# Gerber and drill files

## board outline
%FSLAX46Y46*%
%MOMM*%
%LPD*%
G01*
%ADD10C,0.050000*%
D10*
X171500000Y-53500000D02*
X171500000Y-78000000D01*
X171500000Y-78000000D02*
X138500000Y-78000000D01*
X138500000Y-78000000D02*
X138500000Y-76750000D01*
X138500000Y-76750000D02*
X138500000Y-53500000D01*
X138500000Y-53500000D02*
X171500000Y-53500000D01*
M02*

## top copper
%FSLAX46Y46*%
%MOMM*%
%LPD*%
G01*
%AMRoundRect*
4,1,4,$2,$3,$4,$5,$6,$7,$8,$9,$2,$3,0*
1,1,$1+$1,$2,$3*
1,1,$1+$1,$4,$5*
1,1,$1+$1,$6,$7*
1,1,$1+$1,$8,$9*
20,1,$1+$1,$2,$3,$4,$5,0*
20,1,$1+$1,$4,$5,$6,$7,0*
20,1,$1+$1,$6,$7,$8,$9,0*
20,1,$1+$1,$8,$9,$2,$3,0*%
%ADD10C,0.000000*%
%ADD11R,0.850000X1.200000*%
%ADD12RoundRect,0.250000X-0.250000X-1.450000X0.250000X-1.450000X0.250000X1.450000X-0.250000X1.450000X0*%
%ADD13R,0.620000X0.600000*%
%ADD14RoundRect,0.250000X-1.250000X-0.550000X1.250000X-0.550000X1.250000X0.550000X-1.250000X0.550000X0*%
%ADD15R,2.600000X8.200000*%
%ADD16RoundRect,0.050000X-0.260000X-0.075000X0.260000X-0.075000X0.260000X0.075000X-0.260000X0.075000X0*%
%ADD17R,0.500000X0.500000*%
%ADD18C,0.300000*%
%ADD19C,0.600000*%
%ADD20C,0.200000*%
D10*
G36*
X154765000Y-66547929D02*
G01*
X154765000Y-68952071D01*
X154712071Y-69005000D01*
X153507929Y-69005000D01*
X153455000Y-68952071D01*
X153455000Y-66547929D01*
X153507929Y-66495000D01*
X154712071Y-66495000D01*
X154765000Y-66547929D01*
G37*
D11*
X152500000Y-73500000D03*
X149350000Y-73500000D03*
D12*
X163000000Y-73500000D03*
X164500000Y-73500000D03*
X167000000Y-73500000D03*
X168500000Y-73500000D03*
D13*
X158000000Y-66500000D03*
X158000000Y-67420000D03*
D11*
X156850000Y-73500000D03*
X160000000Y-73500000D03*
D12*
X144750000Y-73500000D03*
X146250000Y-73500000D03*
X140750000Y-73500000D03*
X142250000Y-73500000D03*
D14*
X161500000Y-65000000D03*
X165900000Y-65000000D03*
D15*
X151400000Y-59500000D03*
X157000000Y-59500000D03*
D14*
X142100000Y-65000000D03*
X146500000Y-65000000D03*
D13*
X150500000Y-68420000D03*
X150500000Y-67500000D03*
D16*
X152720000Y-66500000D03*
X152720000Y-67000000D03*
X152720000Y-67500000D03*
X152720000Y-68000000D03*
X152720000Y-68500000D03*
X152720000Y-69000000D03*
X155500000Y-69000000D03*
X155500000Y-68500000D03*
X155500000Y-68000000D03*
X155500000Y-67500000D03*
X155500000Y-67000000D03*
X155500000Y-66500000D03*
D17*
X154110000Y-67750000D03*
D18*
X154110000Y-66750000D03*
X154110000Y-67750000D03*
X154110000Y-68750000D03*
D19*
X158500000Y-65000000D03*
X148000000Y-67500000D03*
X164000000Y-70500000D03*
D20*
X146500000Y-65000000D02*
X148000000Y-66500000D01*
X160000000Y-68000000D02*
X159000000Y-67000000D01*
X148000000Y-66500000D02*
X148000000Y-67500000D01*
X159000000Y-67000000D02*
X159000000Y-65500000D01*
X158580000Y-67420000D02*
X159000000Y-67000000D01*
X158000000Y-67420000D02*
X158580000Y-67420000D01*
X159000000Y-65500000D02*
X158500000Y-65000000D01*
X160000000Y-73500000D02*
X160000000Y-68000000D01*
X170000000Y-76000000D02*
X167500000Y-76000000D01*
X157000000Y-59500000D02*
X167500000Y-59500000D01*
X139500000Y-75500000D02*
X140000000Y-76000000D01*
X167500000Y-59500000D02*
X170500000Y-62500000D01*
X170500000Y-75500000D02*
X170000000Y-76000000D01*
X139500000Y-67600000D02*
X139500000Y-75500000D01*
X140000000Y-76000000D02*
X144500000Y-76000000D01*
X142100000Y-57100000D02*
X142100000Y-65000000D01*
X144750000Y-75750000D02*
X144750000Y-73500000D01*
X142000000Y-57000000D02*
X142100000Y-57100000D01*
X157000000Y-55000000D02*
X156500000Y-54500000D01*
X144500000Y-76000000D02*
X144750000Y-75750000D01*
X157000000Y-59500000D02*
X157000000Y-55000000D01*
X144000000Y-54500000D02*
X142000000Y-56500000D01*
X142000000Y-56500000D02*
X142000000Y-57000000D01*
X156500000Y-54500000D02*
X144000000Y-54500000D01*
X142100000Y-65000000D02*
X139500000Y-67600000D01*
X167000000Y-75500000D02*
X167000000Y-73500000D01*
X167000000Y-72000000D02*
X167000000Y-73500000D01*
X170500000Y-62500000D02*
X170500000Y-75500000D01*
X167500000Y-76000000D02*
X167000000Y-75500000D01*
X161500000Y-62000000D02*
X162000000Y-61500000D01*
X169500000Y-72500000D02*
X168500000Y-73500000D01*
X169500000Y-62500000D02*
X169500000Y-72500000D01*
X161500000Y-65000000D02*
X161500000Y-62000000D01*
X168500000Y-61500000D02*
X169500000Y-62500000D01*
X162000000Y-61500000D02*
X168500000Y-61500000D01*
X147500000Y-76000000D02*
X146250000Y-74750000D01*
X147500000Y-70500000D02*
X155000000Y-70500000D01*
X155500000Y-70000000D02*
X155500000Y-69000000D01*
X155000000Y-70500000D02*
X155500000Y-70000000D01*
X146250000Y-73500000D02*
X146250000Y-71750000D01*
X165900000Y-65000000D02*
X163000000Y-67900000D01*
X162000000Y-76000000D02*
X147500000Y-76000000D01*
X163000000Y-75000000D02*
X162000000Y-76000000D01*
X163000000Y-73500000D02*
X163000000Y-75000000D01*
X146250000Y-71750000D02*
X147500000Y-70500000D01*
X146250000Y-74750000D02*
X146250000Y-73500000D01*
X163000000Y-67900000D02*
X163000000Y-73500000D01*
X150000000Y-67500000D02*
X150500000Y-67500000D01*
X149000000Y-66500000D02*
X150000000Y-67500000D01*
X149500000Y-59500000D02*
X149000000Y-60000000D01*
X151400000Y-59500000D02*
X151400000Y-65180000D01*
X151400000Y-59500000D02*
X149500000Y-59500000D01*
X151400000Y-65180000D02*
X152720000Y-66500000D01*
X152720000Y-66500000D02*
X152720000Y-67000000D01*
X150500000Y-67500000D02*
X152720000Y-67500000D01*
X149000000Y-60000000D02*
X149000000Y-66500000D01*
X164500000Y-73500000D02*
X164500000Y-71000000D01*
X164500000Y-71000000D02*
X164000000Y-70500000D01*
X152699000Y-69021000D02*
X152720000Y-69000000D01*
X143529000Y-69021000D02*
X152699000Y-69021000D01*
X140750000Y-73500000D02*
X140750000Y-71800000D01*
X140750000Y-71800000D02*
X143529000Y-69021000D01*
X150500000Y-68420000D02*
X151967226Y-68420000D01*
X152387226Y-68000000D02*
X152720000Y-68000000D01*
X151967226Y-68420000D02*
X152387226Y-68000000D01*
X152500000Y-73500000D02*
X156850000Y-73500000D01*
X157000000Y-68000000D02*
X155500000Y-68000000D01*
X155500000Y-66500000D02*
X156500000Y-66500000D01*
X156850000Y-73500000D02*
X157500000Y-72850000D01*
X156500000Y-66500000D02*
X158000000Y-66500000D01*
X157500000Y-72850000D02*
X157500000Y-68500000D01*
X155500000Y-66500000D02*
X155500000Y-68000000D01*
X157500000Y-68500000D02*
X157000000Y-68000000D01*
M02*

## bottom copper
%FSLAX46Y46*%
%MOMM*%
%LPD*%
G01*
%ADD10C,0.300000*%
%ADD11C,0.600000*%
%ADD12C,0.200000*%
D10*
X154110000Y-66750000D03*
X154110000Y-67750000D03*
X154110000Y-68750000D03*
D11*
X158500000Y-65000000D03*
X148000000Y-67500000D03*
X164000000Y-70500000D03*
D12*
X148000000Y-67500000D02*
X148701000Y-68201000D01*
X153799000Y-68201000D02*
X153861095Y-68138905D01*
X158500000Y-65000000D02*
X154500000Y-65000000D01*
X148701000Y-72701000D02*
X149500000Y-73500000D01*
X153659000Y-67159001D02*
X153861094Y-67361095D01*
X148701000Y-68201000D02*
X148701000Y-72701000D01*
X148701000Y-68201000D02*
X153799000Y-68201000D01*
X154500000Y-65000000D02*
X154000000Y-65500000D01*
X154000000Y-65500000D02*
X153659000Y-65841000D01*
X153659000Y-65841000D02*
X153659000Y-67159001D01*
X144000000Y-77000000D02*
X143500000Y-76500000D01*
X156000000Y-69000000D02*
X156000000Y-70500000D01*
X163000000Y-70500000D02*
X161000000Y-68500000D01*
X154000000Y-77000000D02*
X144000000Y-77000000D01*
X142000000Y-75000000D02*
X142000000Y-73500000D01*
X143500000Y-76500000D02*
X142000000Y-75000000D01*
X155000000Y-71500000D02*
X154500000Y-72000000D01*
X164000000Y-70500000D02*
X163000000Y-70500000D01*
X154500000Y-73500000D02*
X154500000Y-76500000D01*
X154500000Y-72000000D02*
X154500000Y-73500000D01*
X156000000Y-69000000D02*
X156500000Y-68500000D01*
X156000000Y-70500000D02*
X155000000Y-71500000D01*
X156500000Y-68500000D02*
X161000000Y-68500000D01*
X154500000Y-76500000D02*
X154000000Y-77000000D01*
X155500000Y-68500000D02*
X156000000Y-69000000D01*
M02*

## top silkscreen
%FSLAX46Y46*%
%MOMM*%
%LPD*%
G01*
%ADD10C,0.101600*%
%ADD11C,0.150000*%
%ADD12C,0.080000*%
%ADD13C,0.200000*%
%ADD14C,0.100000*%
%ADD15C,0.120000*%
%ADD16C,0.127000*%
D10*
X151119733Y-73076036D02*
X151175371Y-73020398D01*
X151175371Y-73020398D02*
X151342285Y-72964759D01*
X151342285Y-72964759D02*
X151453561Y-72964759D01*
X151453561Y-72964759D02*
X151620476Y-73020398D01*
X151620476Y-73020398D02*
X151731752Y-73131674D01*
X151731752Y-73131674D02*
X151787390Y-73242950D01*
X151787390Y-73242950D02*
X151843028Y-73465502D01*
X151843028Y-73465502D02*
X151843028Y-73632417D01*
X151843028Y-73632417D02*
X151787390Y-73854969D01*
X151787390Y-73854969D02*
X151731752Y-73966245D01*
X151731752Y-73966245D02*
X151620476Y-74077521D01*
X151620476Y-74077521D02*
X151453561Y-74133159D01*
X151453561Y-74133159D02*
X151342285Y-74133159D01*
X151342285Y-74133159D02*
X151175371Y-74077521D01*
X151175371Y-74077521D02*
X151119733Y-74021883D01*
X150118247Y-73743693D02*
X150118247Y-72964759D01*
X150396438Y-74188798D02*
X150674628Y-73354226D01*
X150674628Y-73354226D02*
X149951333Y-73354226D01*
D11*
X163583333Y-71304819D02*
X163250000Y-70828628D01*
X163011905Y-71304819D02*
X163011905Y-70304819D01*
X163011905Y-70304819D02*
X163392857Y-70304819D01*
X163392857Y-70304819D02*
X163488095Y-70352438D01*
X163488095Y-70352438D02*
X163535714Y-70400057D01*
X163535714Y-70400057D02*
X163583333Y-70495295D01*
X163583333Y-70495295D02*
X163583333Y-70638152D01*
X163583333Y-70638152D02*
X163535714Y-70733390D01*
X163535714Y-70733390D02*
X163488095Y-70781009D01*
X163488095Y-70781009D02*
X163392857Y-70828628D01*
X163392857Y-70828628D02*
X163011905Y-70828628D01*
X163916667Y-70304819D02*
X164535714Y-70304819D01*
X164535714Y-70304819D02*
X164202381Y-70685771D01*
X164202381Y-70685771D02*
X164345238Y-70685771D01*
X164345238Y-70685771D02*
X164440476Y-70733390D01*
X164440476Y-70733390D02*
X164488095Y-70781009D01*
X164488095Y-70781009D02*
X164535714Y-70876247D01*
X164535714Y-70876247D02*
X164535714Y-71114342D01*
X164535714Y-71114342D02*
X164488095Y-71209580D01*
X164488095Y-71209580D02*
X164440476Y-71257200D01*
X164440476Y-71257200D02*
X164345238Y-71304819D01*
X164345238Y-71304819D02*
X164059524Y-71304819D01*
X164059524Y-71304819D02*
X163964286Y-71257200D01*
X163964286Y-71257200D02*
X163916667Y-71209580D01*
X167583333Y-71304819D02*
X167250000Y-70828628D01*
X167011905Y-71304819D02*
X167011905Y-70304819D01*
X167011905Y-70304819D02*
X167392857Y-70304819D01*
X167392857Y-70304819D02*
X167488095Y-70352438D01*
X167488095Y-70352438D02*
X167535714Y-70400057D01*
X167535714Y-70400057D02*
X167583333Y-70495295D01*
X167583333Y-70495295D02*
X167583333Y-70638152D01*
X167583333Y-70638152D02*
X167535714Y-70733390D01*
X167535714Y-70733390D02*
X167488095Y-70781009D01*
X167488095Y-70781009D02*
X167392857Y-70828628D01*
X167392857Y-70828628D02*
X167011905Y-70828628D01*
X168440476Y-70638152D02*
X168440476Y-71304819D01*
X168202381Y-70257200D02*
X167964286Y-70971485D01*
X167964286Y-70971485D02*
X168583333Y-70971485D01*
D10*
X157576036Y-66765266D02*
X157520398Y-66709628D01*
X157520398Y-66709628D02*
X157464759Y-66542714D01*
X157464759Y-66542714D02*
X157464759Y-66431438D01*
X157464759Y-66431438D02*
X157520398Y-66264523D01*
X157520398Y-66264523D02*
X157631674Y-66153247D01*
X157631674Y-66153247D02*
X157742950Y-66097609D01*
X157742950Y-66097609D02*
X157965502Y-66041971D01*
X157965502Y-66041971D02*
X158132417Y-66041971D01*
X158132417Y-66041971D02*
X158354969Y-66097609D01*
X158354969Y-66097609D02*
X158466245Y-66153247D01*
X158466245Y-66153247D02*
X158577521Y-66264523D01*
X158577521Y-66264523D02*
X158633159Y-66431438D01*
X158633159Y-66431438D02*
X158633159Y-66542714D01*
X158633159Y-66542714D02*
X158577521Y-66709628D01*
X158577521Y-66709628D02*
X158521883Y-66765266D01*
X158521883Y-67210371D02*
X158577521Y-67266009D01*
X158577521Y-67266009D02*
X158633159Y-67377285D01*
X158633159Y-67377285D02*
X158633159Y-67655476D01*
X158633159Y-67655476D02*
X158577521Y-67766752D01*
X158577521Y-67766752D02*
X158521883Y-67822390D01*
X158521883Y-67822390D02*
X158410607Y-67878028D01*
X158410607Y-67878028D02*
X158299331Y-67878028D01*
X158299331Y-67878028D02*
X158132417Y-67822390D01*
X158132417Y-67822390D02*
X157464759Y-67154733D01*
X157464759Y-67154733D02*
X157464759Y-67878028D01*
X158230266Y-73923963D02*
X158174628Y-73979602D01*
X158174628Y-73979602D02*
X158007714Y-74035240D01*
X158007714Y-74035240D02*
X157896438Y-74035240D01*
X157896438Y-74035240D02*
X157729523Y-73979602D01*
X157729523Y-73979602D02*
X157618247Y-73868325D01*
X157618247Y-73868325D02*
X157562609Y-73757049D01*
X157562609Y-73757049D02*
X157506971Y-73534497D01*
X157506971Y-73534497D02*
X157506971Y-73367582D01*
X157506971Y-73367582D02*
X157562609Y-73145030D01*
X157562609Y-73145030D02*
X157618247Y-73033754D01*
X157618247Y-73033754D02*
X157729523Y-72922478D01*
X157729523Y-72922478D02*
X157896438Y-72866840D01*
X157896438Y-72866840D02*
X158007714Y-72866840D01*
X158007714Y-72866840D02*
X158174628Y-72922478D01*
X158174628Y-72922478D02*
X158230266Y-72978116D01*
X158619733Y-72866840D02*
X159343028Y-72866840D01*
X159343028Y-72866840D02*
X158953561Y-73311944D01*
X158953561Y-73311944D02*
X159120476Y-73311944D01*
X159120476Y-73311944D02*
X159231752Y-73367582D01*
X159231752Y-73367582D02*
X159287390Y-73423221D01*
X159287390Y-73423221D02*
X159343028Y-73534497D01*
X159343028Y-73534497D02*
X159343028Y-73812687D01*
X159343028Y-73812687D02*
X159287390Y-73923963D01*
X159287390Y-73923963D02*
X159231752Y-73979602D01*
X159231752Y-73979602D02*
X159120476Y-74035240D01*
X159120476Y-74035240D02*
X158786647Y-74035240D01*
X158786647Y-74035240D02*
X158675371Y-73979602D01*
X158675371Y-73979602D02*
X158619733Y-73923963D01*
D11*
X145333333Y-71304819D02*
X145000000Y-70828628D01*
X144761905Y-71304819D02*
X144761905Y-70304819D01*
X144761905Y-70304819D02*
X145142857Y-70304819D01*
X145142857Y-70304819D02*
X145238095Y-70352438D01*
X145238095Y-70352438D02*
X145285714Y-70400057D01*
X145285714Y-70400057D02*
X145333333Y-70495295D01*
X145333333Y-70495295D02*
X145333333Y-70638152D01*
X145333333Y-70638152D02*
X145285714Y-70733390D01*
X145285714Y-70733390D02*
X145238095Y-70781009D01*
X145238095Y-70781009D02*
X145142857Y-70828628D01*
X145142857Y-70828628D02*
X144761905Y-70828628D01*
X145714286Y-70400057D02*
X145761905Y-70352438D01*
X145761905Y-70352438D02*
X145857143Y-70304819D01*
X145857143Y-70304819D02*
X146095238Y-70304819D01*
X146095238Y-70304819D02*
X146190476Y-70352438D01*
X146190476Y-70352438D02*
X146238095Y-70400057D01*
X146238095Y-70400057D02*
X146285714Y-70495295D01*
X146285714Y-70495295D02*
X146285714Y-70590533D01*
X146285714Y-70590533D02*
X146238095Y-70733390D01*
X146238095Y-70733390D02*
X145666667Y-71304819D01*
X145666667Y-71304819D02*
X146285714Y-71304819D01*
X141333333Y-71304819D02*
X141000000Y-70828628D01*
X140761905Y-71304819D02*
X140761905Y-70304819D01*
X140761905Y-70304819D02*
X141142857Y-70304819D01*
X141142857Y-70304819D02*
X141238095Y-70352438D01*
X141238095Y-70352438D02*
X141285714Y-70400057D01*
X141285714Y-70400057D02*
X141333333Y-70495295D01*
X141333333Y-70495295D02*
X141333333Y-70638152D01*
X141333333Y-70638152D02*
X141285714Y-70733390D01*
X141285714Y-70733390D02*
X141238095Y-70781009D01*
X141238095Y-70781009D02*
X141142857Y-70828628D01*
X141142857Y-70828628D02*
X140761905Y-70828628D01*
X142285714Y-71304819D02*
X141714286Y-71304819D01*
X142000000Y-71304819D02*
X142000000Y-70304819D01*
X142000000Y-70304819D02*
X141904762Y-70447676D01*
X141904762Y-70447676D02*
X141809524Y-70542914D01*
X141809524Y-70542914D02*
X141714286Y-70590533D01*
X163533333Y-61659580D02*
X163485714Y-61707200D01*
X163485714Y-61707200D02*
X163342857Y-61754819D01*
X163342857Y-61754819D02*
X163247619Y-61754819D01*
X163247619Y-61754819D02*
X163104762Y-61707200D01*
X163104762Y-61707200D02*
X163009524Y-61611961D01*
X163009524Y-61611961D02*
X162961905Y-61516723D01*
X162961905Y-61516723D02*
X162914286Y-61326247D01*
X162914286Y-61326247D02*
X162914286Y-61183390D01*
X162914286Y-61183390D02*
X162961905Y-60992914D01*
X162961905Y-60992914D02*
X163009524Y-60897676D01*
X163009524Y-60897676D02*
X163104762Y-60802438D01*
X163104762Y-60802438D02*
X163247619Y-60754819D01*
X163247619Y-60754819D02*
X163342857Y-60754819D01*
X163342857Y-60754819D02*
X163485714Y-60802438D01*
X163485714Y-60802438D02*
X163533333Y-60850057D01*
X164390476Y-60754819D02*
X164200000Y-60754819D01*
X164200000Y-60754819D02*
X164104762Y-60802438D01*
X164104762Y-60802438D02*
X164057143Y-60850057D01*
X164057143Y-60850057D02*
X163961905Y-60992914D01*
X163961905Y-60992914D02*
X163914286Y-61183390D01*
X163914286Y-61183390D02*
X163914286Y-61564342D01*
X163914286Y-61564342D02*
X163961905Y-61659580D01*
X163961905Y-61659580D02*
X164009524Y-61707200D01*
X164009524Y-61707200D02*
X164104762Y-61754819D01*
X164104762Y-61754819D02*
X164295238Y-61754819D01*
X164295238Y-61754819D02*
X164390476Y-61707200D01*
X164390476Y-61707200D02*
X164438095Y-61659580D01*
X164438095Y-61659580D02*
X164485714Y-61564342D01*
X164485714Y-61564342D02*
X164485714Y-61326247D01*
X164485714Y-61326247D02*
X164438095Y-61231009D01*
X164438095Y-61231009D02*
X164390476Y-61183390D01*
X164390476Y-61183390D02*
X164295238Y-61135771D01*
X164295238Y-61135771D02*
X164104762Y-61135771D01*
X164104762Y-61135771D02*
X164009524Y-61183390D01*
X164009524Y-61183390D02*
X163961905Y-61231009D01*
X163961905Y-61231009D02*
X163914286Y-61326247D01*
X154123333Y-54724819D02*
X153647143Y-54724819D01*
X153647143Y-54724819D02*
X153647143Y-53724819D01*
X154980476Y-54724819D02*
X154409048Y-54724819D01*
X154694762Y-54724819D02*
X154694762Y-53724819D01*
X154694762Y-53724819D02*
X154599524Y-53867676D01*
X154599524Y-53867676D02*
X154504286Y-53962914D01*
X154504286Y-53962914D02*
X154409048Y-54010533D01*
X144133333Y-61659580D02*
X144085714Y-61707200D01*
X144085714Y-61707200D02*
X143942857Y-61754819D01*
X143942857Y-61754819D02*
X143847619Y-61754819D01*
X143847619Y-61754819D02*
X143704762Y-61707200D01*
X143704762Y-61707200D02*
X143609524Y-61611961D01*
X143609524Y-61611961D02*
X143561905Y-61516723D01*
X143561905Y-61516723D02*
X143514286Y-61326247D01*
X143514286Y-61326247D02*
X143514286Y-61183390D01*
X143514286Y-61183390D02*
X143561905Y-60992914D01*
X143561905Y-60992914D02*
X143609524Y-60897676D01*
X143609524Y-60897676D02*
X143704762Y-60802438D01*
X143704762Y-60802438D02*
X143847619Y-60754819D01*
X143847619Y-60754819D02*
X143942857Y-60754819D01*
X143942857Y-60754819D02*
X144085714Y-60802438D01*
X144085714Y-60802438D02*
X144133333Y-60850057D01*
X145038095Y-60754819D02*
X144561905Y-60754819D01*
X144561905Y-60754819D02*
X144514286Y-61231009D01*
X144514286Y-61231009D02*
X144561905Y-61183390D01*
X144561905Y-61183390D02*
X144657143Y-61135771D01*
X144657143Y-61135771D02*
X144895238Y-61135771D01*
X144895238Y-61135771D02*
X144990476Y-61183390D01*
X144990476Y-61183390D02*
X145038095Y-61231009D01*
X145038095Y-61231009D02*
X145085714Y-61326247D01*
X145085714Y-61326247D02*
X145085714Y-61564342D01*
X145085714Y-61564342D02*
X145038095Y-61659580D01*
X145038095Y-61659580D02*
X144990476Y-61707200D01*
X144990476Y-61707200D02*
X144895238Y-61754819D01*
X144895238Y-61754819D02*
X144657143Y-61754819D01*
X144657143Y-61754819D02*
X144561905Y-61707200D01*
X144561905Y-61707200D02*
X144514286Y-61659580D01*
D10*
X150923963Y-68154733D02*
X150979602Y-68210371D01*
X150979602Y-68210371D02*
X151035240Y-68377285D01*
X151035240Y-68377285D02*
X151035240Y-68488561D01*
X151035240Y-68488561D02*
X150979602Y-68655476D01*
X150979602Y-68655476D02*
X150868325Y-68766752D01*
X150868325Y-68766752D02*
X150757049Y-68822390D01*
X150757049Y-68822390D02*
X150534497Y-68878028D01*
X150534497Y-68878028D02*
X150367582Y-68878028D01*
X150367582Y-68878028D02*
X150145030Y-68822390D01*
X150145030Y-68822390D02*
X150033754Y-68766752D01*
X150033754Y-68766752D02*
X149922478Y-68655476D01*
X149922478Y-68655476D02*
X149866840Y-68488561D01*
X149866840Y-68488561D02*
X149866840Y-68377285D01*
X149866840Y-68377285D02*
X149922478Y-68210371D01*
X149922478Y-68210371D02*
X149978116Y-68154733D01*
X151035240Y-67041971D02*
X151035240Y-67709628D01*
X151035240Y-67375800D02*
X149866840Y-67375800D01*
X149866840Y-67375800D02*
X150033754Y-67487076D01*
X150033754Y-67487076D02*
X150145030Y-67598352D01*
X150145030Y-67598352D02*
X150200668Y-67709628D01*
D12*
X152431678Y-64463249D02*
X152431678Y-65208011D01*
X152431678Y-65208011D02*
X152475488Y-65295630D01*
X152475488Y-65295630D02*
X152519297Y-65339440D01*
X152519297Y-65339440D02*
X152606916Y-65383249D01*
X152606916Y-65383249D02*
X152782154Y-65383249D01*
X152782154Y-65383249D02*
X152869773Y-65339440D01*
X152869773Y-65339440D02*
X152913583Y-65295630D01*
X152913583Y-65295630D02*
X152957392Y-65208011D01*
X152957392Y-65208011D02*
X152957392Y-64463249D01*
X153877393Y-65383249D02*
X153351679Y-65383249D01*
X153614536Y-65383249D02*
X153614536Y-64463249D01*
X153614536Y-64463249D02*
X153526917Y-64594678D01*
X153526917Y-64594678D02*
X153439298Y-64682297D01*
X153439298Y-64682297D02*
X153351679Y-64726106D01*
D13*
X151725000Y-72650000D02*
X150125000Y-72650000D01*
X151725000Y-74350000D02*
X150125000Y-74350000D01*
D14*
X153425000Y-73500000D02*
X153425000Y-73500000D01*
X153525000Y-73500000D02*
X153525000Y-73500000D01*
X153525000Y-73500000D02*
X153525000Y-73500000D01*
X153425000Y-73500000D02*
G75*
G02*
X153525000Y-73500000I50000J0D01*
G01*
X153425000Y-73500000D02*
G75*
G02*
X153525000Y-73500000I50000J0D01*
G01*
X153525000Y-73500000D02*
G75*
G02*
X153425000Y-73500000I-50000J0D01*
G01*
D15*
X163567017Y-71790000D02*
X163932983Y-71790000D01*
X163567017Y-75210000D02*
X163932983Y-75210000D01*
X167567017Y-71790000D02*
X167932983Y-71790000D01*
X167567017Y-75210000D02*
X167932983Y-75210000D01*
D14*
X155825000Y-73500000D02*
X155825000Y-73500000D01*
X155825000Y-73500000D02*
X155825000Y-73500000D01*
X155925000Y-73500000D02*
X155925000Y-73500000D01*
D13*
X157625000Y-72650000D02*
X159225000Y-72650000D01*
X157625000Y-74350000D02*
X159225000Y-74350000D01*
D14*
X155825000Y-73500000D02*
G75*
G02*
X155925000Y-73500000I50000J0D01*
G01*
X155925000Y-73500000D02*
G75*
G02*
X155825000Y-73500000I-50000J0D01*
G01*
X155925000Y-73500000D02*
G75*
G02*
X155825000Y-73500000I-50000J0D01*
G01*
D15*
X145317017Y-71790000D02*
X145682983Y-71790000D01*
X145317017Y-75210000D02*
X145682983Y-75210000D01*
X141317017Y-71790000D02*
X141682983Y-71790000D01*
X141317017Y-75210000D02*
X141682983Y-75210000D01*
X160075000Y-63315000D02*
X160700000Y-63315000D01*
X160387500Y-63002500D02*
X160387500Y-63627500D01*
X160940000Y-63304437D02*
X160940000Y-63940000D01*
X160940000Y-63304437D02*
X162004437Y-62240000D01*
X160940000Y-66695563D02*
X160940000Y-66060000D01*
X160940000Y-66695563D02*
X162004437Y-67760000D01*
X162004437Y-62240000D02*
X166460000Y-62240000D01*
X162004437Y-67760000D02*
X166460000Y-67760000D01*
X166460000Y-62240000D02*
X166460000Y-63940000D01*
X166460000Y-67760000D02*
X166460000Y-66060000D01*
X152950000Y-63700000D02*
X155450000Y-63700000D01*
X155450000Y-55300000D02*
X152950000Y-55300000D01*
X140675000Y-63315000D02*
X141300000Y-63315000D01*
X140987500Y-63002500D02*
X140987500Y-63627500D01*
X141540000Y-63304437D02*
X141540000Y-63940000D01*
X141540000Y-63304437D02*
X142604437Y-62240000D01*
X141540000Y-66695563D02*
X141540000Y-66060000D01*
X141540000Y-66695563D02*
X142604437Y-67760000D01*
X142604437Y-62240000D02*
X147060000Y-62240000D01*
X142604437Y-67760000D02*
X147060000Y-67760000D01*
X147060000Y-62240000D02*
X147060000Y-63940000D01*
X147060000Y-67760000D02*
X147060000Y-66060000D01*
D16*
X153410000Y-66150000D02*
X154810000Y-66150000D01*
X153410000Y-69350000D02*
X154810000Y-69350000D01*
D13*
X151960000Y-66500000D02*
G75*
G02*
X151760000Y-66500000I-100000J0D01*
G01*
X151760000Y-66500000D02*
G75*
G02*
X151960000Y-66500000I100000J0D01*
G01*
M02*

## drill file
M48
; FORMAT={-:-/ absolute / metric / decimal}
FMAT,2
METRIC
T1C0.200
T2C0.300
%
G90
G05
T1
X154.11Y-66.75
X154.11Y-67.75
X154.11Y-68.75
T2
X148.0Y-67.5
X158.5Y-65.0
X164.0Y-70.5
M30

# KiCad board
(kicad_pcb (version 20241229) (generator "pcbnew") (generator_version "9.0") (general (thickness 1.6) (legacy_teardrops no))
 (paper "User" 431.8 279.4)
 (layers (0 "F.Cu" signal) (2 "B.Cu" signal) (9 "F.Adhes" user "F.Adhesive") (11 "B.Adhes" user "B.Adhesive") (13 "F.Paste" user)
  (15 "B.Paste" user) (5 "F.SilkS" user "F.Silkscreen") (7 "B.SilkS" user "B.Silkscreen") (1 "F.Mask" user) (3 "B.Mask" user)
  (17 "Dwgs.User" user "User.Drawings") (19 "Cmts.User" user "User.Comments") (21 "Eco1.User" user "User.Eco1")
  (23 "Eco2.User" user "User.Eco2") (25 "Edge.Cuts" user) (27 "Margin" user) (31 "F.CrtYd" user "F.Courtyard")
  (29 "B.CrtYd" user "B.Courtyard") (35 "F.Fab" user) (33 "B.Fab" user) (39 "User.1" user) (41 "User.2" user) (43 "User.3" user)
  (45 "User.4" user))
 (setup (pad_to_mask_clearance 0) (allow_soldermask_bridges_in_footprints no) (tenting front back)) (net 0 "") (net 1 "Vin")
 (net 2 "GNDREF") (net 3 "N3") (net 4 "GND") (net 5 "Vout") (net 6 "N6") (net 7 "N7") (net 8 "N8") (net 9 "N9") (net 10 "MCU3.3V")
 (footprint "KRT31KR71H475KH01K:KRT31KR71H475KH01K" (layer "F.Cu") (at 150.925 73.5 180)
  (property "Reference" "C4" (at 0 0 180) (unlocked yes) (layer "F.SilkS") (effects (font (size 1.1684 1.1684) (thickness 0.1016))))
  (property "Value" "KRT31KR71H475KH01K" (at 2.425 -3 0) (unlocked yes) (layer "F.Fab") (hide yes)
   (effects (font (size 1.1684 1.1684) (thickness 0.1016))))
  (fp_line (start -0.8 0.85) (end 0.8 0.85) (stroke (width 0.2) (type solid)) (layer "F.SilkS"))
  (fp_line (start -0.8 -0.85) (end 0.8 -0.85) (stroke (width 0.2) (type solid)) (layer "F.SilkS"))
  (fp_line (start -2.5 0) (end -2.5 0) (stroke (width 0.1) (type solid)) (layer "F.SilkS"))
  (fp_line (start -2.6 0) (end -2.6 0) (stroke (width 0.1) (type solid)) (layer "F.SilkS"))
  (fp_line (start -2.6 0) (end -2.6 0) (stroke (width 0.1) (type solid)) (layer "F.SilkS"))
  (fp_arc (start -2.5 0) (mid -2.55 0.05) (end -2.6 0) (stroke (width 0.1) (type solid)) (layer "F.SilkS"))
  (fp_arc (start -2.5 0) (mid -2.55 0.05) (end -2.6 0) (stroke (width 0.1) (type solid)) (layer "F.SilkS"))
  (fp_arc (start -2.6 0) (mid -2.55 -0.05) (end -2.5 0) (stroke (width 0.1) (type solid)) (layer "F.SilkS"))
  (pad "1" smd rect (at -1.575 0 270) (size 1.2 0.85) (layers "F.Cu" "F.Mask" "F.Paste") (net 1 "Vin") (solder_mask_margin 0.1016)
   (solder_paste_margin 0) (thermal_bridge_angle 0))
  (pad "2" smd rect (at 1.575 0 270) (size 1.2 0.85) (layers "F.Cu" "F.Mask" "F.Paste") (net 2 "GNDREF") (solder_mask_margin 0.1016)
   (solder_paste_margin 0) (thermal_bridge_angle 0)))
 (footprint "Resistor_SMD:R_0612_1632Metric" (layer "F.Cu") (at 163.75 73.5)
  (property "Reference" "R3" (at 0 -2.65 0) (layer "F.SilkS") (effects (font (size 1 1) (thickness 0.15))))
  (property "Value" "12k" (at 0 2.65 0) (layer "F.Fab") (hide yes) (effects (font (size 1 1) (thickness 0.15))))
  (fp_line (start -0.182983 -1.71) (end 0.182983 -1.71) (stroke (width 0.12) (type solid)) (layer "F.SilkS"))
  (fp_line (start -0.182983 1.71) (end 0.182983 1.71) (stroke (width 0.12) (type solid)) (layer "F.SilkS"))
  (pad "1" smd roundrect (at -0.75 0) (size 1 3.4) (layers "F.Cu" "F.Mask" "F.Paste") (roundrect_rratio 0.25) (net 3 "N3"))
  (pad "2" smd roundrect (at 0.75 0) (size 1 3.4) (layers "F.Cu" "F.Mask" "F.Paste") (roundrect_rratio 0.25) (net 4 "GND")))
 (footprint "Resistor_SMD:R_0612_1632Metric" (layer "F.Cu") (at 167.75 73.5)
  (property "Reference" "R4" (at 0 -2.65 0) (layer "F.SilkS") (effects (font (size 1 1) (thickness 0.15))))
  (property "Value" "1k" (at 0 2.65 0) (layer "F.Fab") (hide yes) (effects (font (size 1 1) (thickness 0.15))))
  (fp_line (start -0.182983 -1.71) (end 0.182983 -1.71) (stroke (width 0.12) (type solid)) (layer "F.SilkS"))
  (fp_line (start -0.182983 1.71) (end 0.182983 1.71) (stroke (width 0.12) (type solid)) (layer "F.SilkS"))
  (pad "1" smd roundrect (at -0.75 0) (size 1 3.4) (layers "F.Cu" "F.Mask" "F.Paste") (roundrect_rratio 0.25) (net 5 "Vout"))
  (pad "2" smd roundrect (at 0.75 0) (size 1 3.4) (layers "F.Cu" "F.Mask" "F.Paste") (roundrect_rratio 0.25) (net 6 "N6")))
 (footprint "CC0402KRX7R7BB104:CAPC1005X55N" (layer "F.Cu") (at 158 66.96 -90)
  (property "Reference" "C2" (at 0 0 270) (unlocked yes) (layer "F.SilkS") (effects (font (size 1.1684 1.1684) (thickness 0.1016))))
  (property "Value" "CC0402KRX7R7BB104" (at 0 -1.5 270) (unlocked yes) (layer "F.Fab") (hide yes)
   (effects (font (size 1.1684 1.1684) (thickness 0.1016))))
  (pad "1" smd rect (at -0.46 0) (size 0.62 0.6) (layers "F.Cu" "F.Mask" "F.Paste") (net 1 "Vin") (solder_mask_margin 0.1016)
   (solder_paste_margin 0) (thermal_bridge_angle 0))
  (pad "2" smd rect (at 0.46 0) (size 0.62 0.6) (layers "F.Cu" "F.Mask" "F.Paste") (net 2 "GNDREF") (solder_mask_margin 0.1016)
   (solder_paste_margin 0) (thermal_bridge_angle 0)))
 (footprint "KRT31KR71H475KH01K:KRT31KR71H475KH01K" (layer "F.Cu") (at 158.425 73.5)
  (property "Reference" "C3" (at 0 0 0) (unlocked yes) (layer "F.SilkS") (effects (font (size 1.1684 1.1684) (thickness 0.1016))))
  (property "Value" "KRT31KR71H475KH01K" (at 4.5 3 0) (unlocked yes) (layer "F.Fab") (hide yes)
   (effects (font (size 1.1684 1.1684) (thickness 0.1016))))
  (fp_line (start -2.6 0) (end -2.6 0) (stroke (width 0.1) (type solid)) (layer "F.SilkS"))
  (fp_line (start -2.6 0) (end -2.6 0) (stroke (width 0.1) (type solid)) (layer "F.SilkS"))
  (fp_line (start -2.5 0) (end -2.5 0) (stroke (width 0.1) (type solid)) (layer "F.SilkS"))
  (fp_line (start -0.8 -0.85) (end 0.8 -0.85) (stroke (width 0.2) (type solid)) (layer "F.SilkS"))
  (fp_line (start -0.8 0.85) (end 0.8 0.85) (stroke (width 0.2) (type solid)) (layer "F.SilkS"))
  (fp_arc (start -2.6 0) (mid -2.55 -0.05) (end -2.5 0) (stroke (width 0.1) (type solid)) (layer "F.SilkS"))
  (fp_arc (start -2.5 0) (mid -2.55 0.05) (end -2.6 0) (stroke (width 0.1) (type solid)) (layer "F.SilkS"))
  (fp_arc (start -2.5 0) (mid -2.55 0.05) (end -2.6 0) (stroke (width 0.1) (type solid)) (layer "F.SilkS"))
  (pad "1" smd rect (at -1.575 0 90) (size 1.2 0.85) (layers "F.Cu" "F.Mask" "F.Paste") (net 1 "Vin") (solder_mask_margin 0.1016)
   (solder_paste_margin 0) (thermal_bridge_angle 0))
  (pad "2" smd rect (at 1.575 0 90) (size 1.2 0.85) (layers "F.Cu" "F.Mask" "F.Paste") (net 2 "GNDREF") (solder_mask_margin 0.1016)
   (solder_paste_margin 0) (thermal_bridge_angle 0)))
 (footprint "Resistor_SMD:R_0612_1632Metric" (layer "F.Cu") (at 145.5 73.5)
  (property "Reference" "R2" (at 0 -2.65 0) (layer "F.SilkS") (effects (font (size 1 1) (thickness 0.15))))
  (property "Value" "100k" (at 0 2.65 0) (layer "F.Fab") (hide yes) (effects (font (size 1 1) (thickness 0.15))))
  (fp_line (start -0.182983 -1.71) (end 0.182983 -1.71) (stroke (width 0.12) (type solid)) (layer "F.SilkS"))
  (fp_line (start -0.182983 1.71) (end 0.182983 1.71) (stroke (width 0.12) (type solid)) (layer "F.SilkS"))
  (pad "1" smd roundrect (at -0.75 0) (size 1 3.4) (layers "F.Cu" "F.Mask" "F.Paste") (roundrect_rratio 0.25) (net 5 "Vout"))
  (pad "2" smd roundrect (at 0.75 0) (size 1 3.4) (layers "F.Cu" "F.Mask" "F.Paste") (roundrect_rratio 0.25) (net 3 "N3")))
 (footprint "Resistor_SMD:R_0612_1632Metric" (layer "F.Cu") (at 141.5 73.5)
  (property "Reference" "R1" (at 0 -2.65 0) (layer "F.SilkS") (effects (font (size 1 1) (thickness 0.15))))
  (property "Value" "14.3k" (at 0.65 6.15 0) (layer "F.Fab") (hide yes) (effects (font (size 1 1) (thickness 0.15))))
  (fp_line (start -0.182983 -1.71) (end 0.182983 -1.71) (stroke (width 0.12) (type solid)) (layer "F.SilkS"))
  (fp_line (start -0.182983 1.71) (end 0.182983 1.71) (stroke (width 0.12) (type solid)) (layer "F.SilkS"))
  (pad "1" smd roundrect (at -0.75 0) (size 1 3.4) (layers "F.Cu" "F.Mask" "F.Paste") (roundrect_rratio 0.25) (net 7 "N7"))
  (pad "2" smd roundrect (at 0.75 0) (size 1 3.4) (layers "F.Cu" "F.Mask" "F.Paste") (roundrect_rratio 0.25) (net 4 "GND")))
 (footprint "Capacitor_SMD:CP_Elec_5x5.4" (layer "F.Cu") (at 163.7 65)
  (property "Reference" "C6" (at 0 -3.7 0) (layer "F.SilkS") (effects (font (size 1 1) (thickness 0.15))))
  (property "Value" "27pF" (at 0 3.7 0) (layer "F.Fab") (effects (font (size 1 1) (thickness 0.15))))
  (fp_line (start -3.625 -1.685) (end -3 -1.685) (stroke (width 0.12) (type solid)) (layer "F.SilkS"))
  (fp_line (start -3.3125 -1.9975) (end -3.3125 -1.3725) (stroke (width 0.12) (type solid)) (layer "F.SilkS"))
  (fp_line (start -2.76 -1.695563) (end -2.76 -1.06) (stroke (width 0.12) (type solid)) (layer "F.SilkS"))
  (fp_line (start -2.76 -1.695563) (end -1.695563 -2.76) (stroke (width 0.12) (type solid)) (layer "F.SilkS"))
  (fp_line (start -2.76 1.695563) (end -2.76 1.06) (stroke (width 0.12) (type solid)) (layer "F.SilkS"))
  (fp_line (start -2.76 1.695563) (end -1.695563 2.76) (stroke (width 0.12) (type solid)) (layer "F.SilkS"))
  (fp_line (start -1.695563 -2.76) (end 2.76 -2.76) (stroke (width 0.12) (type solid)) (layer "F.SilkS"))
  (fp_line (start -1.695563 2.76) (end 2.76 2.76) (stroke (width 0.12) (type solid)) (layer "F.SilkS"))
  (fp_line (start 2.76 -2.76) (end 2.76 -1.06) (stroke (width 0.12) (type solid)) (layer "F.SilkS"))
  (fp_line (start 2.76 2.76) (end 2.76 1.06) (stroke (width 0.12) (type solid)) (layer "F.SilkS"))
  (pad "1" smd roundrect (at -2.2 0) (size 3 1.6) (layers "F.Cu" "F.Mask" "F.Paste") (roundrect_rratio 0.15625) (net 6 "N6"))
  (pad "2" smd roundrect (at 2.2 0) (size 3 1.6) (layers "F.Cu" "F.Mask" "F.Paste") (roundrect_rratio 0.15625) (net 3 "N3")))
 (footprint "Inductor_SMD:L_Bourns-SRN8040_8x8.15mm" (layer "F.Cu") (at 154.2 59.5)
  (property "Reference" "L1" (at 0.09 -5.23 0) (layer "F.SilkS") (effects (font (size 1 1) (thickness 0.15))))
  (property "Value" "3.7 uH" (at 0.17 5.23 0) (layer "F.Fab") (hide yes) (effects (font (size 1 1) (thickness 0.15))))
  (fp_line (start -1.25 4.2) (end 1.25 4.2) (stroke (width 0.12) (type solid)) (layer "F.SilkS"))
  (fp_line (start 1.25 -4.2) (end -1.25 -4.2) (stroke (width 0.12) (type solid)) (layer "F.SilkS"))
  (pad "1" smd rect (at -2.8 0) (size 2.6 8.2) (layers "F.Cu" "F.Mask" "F.Paste") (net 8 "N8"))
  (pad "2" smd rect (at 2.8 0) (size 2.6 8.2) (layers "F.Cu" "F.Mask" "F.Paste") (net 5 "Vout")))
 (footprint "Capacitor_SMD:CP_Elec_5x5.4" (layer "F.Cu") (at 144.3 65)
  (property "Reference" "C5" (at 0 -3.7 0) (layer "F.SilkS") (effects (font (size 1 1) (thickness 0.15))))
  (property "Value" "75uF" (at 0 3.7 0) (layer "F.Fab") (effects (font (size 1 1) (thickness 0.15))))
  (fp_line (start -3.625 -1.685) (end -3 -1.685) (stroke (width 0.12) (type solid)) (layer "F.SilkS"))
  (fp_line (start -3.3125 -1.9975) (end -3.3125 -1.3725) (stroke (width 0.12) (type solid)) (layer "F.SilkS"))
  (fp_line (start -2.76 -1.695563) (end -2.76 -1.06) (stroke (width 0.12) (type solid)) (layer "F.SilkS"))
  (fp_line (start -2.76 -1.695563) (end -1.695563 -2.76) (stroke (width 0.12) (type solid)) (layer "F.SilkS"))
  (fp_line (start -2.76 1.695563) (end -2.76 1.06) (stroke (width 0.12) (type solid)) (layer "F.SilkS"))
  (fp_line (start -2.76 1.695563) (end -1.695563 2.76) (stroke (width 0.12) (type solid)) (layer "F.SilkS"))
  (fp_line (start -1.695563 -2.76) (end 2.76 -2.76) (stroke (width 0.12) (type solid)) (layer "F.SilkS"))
  (fp_line (start -1.695563 2.76) (end 2.76 2.76) (stroke (width 0.12) (type solid)) (layer "F.SilkS"))
  (fp_line (start 2.76 -2.76) (end 2.76 -1.06) (stroke (width 0.12) (type solid)) (layer "F.SilkS"))
  (fp_line (start 2.76 2.76) (end 2.76 1.06) (stroke (width 0.12) (type solid)) (layer "F.SilkS"))
  (pad "1" smd roundrect (at -2.2 0) (size 3 1.6) (layers "F.Cu" "F.Mask" "F.Paste") (roundrect_rratio 0.15625) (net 5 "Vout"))
  (pad "2" smd roundrect (at 2.2 0) (size 3 1.6) (layers "F.Cu" "F.Mask" "F.Paste") (roundrect_rratio 0.15625) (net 2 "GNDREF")))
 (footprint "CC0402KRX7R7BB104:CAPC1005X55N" (layer "F.Cu") (at 150.5 67.96 90)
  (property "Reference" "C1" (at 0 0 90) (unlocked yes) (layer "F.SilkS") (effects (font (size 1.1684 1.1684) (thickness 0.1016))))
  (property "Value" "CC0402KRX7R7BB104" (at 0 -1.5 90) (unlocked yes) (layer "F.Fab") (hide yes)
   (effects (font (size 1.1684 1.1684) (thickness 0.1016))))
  (pad "1" smd rect (at -0.46 0 180) (size 0.62 0.6) (layers "F.Cu" "F.Mask" "F.Paste") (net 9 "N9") (solder_mask_margin 0.1016)
   (solder_paste_margin 0) (thermal_bridge_angle 0))
  (pad "2" smd rect (at 0.46 0 180) (size 0.62 0.6) (layers "F.Cu" "F.Mask" "F.Paste") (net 8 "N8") (solder_mask_margin 0.1016)
   (solder_paste_margin 0) (thermal_bridge_angle 0)))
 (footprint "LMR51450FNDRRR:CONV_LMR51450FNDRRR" (layer "F.Cu") (at 154.11 67.75)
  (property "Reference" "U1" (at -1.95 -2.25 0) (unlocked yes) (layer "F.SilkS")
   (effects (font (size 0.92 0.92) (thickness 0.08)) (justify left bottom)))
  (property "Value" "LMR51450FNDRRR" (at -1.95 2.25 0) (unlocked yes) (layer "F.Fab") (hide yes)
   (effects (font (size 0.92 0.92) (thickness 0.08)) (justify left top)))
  (fp_poly
   (pts (xy 0.655 -1.202071) (xy 0.655 1.202071) (xy 0.602071 1.255) (xy -0.602071 1.255) (xy -0.655 1.202071) (xy -0.655 -1.202071)
    (xy -0.602071 -1.255) (xy 0.602071 -1.255))
   (stroke (width 0) (type default)) (fill yes) (layer "F.Cu"))
  (fp_line (start -0.7 -1.6) (end 0.7 -1.6) (stroke (width 0.127) (type solid)) (layer "F.SilkS"))
  (fp_line (start -0.7 1.6) (end 0.7 1.6) (stroke (width 0.127) (type solid)) (layer "F.SilkS"))
  (fp_circle (center -2.25 -1.25) (end -2.15 -1.25) (stroke (width 0.2) (type solid)) (fill no) (layer "F.SilkS"))
  (pad "1" smd roundrect (at -1.39 -1.25) (size 0.62 0.25) (layers "F.Cu" "F.Paste") (roundrect_rratio 0.2) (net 8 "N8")
   (solder_mask_margin 0.1016) (solder_paste_margin 0) (thermal_bridge_angle 0))
  (pad "2" smd roundrect (at -1.39 -0.75) (size 0.62 0.25) (layers "F.Cu" "F.Paste") (roundrect_rratio 0.2) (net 8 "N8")
   (solder_mask_margin 0.1016) (solder_paste_margin 0) (thermal_bridge_angle 0))
  (pad "3" smd roundrect (at -1.39 -0.25) (size 0.62 0.25) (layers "F.Cu" "F.Paste") (roundrect_rratio 0.2) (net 8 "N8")
   (solder_mask_margin 0.1016) (solder_paste_margin 0) (thermal_bridge_angle 0))
  (pad "4" smd roundrect (at -1.39 0.25) (size 0.62 0.25) (layers "F.Cu" "F.Paste") (roundrect_rratio 0.2) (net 9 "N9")
   (solder_mask_margin 0.1016) (solder_paste_margin 0) (thermal_bridge_angle 0))
  (pad "5" smd roundrect (at -1.39 0.75) (size 0.62 0.25) (layers "F.Cu" "F.Paste") (roundrect_rratio 0.2) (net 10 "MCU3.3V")
   (solder_mask_margin 0.1016) (solder_paste_margin 0) (thermal_bridge_angle 0))
  (pad "6" smd roundrect (at -1.39 1.25) (size 0.62 0.25) (layers "F.Cu" "F.Paste") (roundrect_rratio 0.2) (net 7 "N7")
   (solder_mask_margin 0.1016) (solder_paste_margin 0) (thermal_bridge_angle 0))
  (pad "7" smd roundrect (at 1.39 1.25) (size 0.62 0.25) (layers "F.Cu" "F.Paste") (roundrect_rratio 0.2) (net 3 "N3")
   (solder_mask_margin 0.1016) (solder_paste_margin 0) (thermal_bridge_angle 0))
  (pad "8" smd roundrect (at 1.39 0.75) (size 0.62 0.25) (layers "F.Cu" "F.Paste") (roundrect_rratio 0.2) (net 4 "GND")
   (solder_mask_margin 0.1016) (solder_paste_margin 0) (thermal_bridge_angle 0))
  (pad "9" smd roundrect (at 1.39 0.25) (size 0.62 0.25) (layers "F.Cu" "F.Paste") (roundrect_rratio 0.2) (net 1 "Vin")
   (solder_mask_margin 0.1016) (solder_paste_margin 0) (thermal_bridge_angle 0))
  (pad "10" smd roundrect (at 1.39 -0.25) (size 0.62 0.25) (layers "F.Cu" "F.Paste") (roundrect_rratio 0.2) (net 1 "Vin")
   (solder_mask_margin 0.1016) (solder_paste_margin 0) (thermal_bridge_angle 0))
  (pad "11" smd roundrect (at 1.39 -0.75) (size 0.62 0.25) (layers "F.Cu" "F.Paste") (roundrect_rratio 0.2) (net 1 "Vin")
   (solder_mask_margin 0.1016) (solder_paste_margin 0) (thermal_bridge_angle 0))
  (pad "12" smd roundrect (at 1.39 -1.25) (size 0.62 0.25) (layers "F.Cu" "F.Paste") (roundrect_rratio 0.2) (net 1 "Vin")
   (solder_mask_margin 0.1016) (solder_paste_margin 0) (thermal_bridge_angle 0))
  (pad "13" smd rect (at 0 0) (size 0.5 0.5) (layers "F.Cu") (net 2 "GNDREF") (solder_mask_margin 0.1016) (solder_paste_margin 0)
   (thermal_bridge_angle 0))
  (pad "14" thru_hole circle (at 0 -1) (size 0.3 0.3) (drill 0.2) (layers "*.Cu") (remove_unused_layers no) (solder_mask_margin 0.1016)
   (thermal_bridge_angle 0))
  (pad "15" thru_hole circle (at 0 0) (size 0.3 0.3) (drill 0.2) (layers "*.Cu") (remove_unused_layers no) (solder_mask_margin 0.1016)
   (thermal_bridge_angle 0))
  (pad "16" thru_hole circle (at 0 1) (size 0.3 0.3) (drill 0.2) (layers "*.Cu") (remove_unused_layers no) (solder_mask_margin 0.1016)
   (thermal_bridge_angle 0)))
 (gr_line (start 171.5 53.5) (end 171.5 78) (stroke (width 0.05) (type default)) (layer "Edge.Cuts"))
 (gr_line (start 171.5 78) (end 138.5 78) (stroke (width 0.05) (type default)) (layer "Edge.Cuts"))
 (gr_line (start 138.5 78) (end 138.5 76.75) (stroke (width 0.05) (type default)) (layer "Edge.Cuts"))
 (gr_line (start 138.5 76.75) (end 138.5 53.5) (stroke (width 0.05) (type default)) (layer "Edge.Cuts"))
 (gr_line (start 138.5 53.5) (end 171.5 53.5) (stroke (width 0.05) (type default)) (layer "Edge.Cuts"))
 (segment (start 146.5 65) (end 148 66.5) (width 0.2) (layer "F.Cu") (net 2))
 (segment (start 160 68) (end 159 67) (width 0.2) (layer "F.Cu") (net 2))
 (segment (start 148 66.5) (end 148 67.5) (width 0.2) (layer "F.Cu") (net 2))
 (segment (start 159 67) (end 159 65.5) (width 0.2) (layer "F.Cu") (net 2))
 (segment (start 158.58 67.42) (end 159 67) (width 0.2) (layer "F.Cu") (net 2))
 (segment (start 158 67.42) (end 158.58 67.42) (width 0.2) (layer "F.Cu") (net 2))
 (segment (start 159 65.5) (end 158.5 65) (width 0.2) (layer "F.Cu") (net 2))
 (segment (start 160 73.5) (end 160 68) (width 0.2) (layer "F.Cu") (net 2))
 (via (at 158.5 65) (size 0.6) (drill 0.3) (layers "F.Cu" "B.Cu") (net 2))
 (via (at 148 67.5) (size 0.6) (drill 0.3) (layers "F.Cu" "B.Cu") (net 2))
 (segment (start 148 67.5) (end 148.701 68.201) (width 0.2) (layer "B.Cu") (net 2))
 (segment (start 153.799 68.201) (end 153.861095 68.138905) (width 0.2) (layer "B.Cu") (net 2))
 (segment (start 158.5 65) (end 154.5 65) (width 0.2) (layer "B.Cu") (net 2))
 (segment (start 148.701 72.701) (end 149.5 73.5) (width 0.2) (layer "B.Cu") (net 2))
 (segment (start 153.659 67.159001) (end 153.861094 67.361095) (width 0.2) (layer "B.Cu") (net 2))
 (segment (start 148.701 68.201) (end 148.701 72.701) (width 0.2) (layer "B.Cu") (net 2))
 (segment (start 148.701 68.201) (end 153.799 68.201) (width 0.2) (layer "B.Cu") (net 2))
 (segment (start 154.5 65) (end 154 65.5) (width 0.2) (layer "B.Cu") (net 2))
 (segment (start 154 65.5) (end 153.659 65.841) (width 0.2) (layer "B.Cu") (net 2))
 (segment (start 153.659 65.841) (end 153.659 67.159001) (width 0.2) (layer "B.Cu") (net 2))
 (segment (start 170 76) (end 167.5 76) (width 0.2) (layer "F.Cu") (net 5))
 (segment (start 157 59.5) (end 167.5 59.5) (width 0.2) (layer "F.Cu") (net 5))
 (segment (start 139.5 75.5) (end 140 76) (width 0.2) (layer "F.Cu") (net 5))
 (segment (start 167.5 59.5) (end 170.5 62.5) (width 0.2) (layer "F.Cu") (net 5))
 (segment (start 170.5 75.5) (end 170 76) (width 0.2) (layer "F.Cu") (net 5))
 (segment (start 139.5 67.6) (end 139.5 75.5) (width 0.2) (layer "F.Cu") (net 5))
 (segment (start 140 76) (end 144.5 76) (width 0.2) (layer "F.Cu") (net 5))
 (segment (start 142.1 57.1) (end 142.1 65) (width 0.2) (layer "F.Cu") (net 5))
 (segment (start 144.75 75.75) (end 144.75 73.5) (width 0.2) (layer "F.Cu") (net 5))
 (segment (start 142 57) (end 142.1 57.1) (width 0.2) (layer "F.Cu") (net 5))
 (segment (start 157 55) (end 156.5 54.5) (width 0.2) (layer "F.Cu") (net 5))
 (segment (start 144.5 76) (end 144.75 75.75) (width 0.2) (layer "F.Cu") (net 5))
 (segment (start 157 59.5) (end 157 55) (width 0.2) (layer "F.Cu") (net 5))
 (segment (start 144 54.5) (end 142 56.5) (width 0.2) (layer "F.Cu") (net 5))
 (segment (start 142 56.5) (end 142 57) (width 0.2) (layer "F.Cu") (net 5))
 (segment (start 156.5 54.5) (end 144 54.5) (width 0.2) (layer "F.Cu") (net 5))
 (segment (start 142.1 65) (end 139.5 67.6) (width 0.2) (layer "F.Cu") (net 5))
 (segment (start 167 75.5) (end 167 73.5) (width 0.2) (layer "F.Cu") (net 5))
 (segment (start 167 72) (end 167 73.5) (width 0.2) (layer "F.Cu") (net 5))
 (segment (start 170.5 62.5) (end 170.5 75.5) (width 0.2) (layer "F.Cu") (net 5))
 (segment (start 167.5 76) (end 167 75.5) (width 0.2) (layer "F.Cu") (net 5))
 (segment (start 161.5 62) (end 162 61.5) (width 0.2) (layer "F.Cu") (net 6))
 (segment (start 169.5 72.5) (end 168.5 73.5) (width 0.2) (layer "F.Cu") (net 6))
 (segment (start 169.5 62.5) (end 169.5 72.5) (width 0.2) (layer "F.Cu") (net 6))
 (segment (start 161.5 65) (end 161.5 62) (width 0.2) (layer "F.Cu") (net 6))
 (segment (start 168.5 61.5) (end 169.5 62.5) (width 0.2) (layer "F.Cu") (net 6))
 (segment (start 162 61.5) (end 168.5 61.5) (width 0.2) (layer "F.Cu") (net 6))
 (segment (start 147.5 76) (end 146.25 74.75) (width 0.2) (layer "F.Cu") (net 3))
 (segment (start 147.5 70.5) (end 155 70.5) (width 0.2) (layer "F.Cu") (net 3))
 (segment (start 155.5 70) (end 155.5 69) (width 0.2) (layer "F.Cu") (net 3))
 (segment (start 155 70.5) (end 155.5 70) (width 0.2) (layer "F.Cu") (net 3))
 (segment (start 146.25 73.5) (end 146.25 71.75) (width 0.2) (layer "F.Cu") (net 3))
 (segment (start 165.9 65) (end 163 67.9) (width 0.2) (layer "F.Cu") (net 3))
 (segment (start 162 76) (end 147.5 76) (width 0.2) (layer "F.Cu") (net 3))
 (segment (start 163 75) (end 162 76) (width 0.2) (layer "F.Cu") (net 3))
 (segment (start 163 73.5) (end 163 75) (width 0.2) (layer "F.Cu") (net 3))
 (segment (start 146.25 71.75) (end 147.5 70.5) (width 0.2) (layer "F.Cu") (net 3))
 (segment (start 146.25 74.75) (end 146.25 73.5) (width 0.2) (layer "F.Cu") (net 3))
 (segment (start 163 67.9) (end 163 73.5) (width 0.2) (layer "F.Cu") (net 3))
 (segment (start 150 67.5) (end 150.5 67.5) (width 0.2) (layer "F.Cu") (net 8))
 (segment (start 149 66.5) (end 150 67.5) (width 0.2) (layer "F.Cu") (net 8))
 (segment (start 149.5 59.5) (end 149 60) (width 0.2) (layer "F.Cu") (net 8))
 (segment (start 151.4 59.5) (end 151.4 65.18) (width 0.2) (layer "F.Cu") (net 8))
 (segment (start 151.4 59.5) (end 149.5 59.5) (width 0.2) (layer "F.Cu") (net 8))
 (segment (start 151.4 65.18) (end 152.72 66.5) (width 0.2) (layer "F.Cu") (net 8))
 (segment (start 152.72 66.5) (end 152.72 67) (width 0.2) (layer "F.Cu") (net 8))
 (segment (start 150.5 67.5) (end 152.72 67.5) (width 0.2) (layer "F.Cu") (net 8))
 (segment (start 149 60) (end 149 66.5) (width 0.2) (layer "F.Cu") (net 8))
 (segment (start 164.5 73.5) (end 164.5 71) (width 0.2) (layer "F.Cu") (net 4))
 (segment (start 164.5 71) (end 164 70.5) (width 0.2) (layer "F.Cu") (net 4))
 (via (at 164 70.5) (size 0.6) (drill 0.3) (layers "F.Cu" "B.Cu") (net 4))
 (segment (start 144 77) (end 143.5 76.5) (width 0.2) (layer "B.Cu") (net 4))
 (segment (start 156 69) (end 156 70.5) (width 0.2) (layer "B.Cu") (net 4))
 (segment (start 163 70.5) (end 161 68.5) (width 0.2) (layer "B.Cu") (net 4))
 (segment (start 154 77) (end 144 77) (width 0.2) (layer "B.Cu") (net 4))
 (segment (start 142 75) (end 142 73.5) (width 0.2) (layer "B.Cu") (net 4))
 (segment (start 143.5 76.5) (end 142 75) (width 0.2) (layer "B.Cu") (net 4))
 (segment (start 155 71.5) (end 154.5 72) (width 0.2) (layer "B.Cu") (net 4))
 (segment (start 164 70.5) (end 163 70.5) (width 0.2) (layer "B.Cu") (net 4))
 (segment (start 154.5 73.5) (end 154.5 76.5) (width 0.2) (layer "B.Cu") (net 4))
 (segment (start 154.5 72) (end 154.5 73.5) (width 0.2) (layer "B.Cu") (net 4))
 (segment (start 156 69) (end 156.5 68.5) (width 0.2) (layer "B.Cu") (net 4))
 (segment (start 156 70.5) (end 155 71.5) (width 0.2) (layer "B.Cu") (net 4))
 (segment (start 156.5 68.5) (end 161 68.5) (width 0.2) (layer "B.Cu") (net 4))
 (segment (start 154.5 76.5) (end 154 77) (width 0.2) (layer "B.Cu") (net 4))
 (segment (start 155.5 68.5) (end 156 69) (width 0.2) (layer "B.Cu") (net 4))
 (segment (start 152.699 69.021) (end 152.72 69) (width 0.2) (layer "F.Cu") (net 7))
 (segment (start 143.529 69.021) (end 152.699 69.021) (width 0.2) (layer "F.Cu") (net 7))
 (segment (start 140.75 73.5) (end 140.75 71.8) (width 0.2) (layer "F.Cu") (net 7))
 (segment (start 140.75 71.8) (end 143.529 69.021) (width 0.2) (layer "F.Cu") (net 7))
 (segment (start 150.5 68.42) (end 151.967226 68.42) (width 0.2) (layer "F.Cu") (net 9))
 (segment (start 152.387226 68) (end 152.72 68) (width 0.2) (layer "F.Cu") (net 9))
 (segment (start 151.967226 68.42) (end 152.387226 68) (width 0.2) (layer "F.Cu") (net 9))
 (segment (start 152.5 73.5) (end 156.85 73.5) (width 0.2) (layer "F.Cu") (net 1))
 (segment (start 157 68) (end 155.5 68) (width 0.2) (layer "F.Cu") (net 1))
 (segment (start 155.5 66.5) (end 156.5 66.5) (width 0.2) (layer "F.Cu") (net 1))
 (segment (start 156.85 73.5) (end 157.5 72.85) (width 0.2) (layer "F.Cu") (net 1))
 (segment (start 156.5 66.5) (end 158 66.5) (width 0.2) (layer "F.Cu") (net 1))
 (segment (start 157.5 72.85) (end 157.5 68.5) (width 0.2) (layer "F.Cu") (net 1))
 (segment (start 155.5 66.5) (end 155.5 68) (width 0.2) (layer "F.Cu") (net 1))
 (segment (start 157.5 68.5) (end 157 68) (width 0.2) (layer "F.Cu") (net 1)))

